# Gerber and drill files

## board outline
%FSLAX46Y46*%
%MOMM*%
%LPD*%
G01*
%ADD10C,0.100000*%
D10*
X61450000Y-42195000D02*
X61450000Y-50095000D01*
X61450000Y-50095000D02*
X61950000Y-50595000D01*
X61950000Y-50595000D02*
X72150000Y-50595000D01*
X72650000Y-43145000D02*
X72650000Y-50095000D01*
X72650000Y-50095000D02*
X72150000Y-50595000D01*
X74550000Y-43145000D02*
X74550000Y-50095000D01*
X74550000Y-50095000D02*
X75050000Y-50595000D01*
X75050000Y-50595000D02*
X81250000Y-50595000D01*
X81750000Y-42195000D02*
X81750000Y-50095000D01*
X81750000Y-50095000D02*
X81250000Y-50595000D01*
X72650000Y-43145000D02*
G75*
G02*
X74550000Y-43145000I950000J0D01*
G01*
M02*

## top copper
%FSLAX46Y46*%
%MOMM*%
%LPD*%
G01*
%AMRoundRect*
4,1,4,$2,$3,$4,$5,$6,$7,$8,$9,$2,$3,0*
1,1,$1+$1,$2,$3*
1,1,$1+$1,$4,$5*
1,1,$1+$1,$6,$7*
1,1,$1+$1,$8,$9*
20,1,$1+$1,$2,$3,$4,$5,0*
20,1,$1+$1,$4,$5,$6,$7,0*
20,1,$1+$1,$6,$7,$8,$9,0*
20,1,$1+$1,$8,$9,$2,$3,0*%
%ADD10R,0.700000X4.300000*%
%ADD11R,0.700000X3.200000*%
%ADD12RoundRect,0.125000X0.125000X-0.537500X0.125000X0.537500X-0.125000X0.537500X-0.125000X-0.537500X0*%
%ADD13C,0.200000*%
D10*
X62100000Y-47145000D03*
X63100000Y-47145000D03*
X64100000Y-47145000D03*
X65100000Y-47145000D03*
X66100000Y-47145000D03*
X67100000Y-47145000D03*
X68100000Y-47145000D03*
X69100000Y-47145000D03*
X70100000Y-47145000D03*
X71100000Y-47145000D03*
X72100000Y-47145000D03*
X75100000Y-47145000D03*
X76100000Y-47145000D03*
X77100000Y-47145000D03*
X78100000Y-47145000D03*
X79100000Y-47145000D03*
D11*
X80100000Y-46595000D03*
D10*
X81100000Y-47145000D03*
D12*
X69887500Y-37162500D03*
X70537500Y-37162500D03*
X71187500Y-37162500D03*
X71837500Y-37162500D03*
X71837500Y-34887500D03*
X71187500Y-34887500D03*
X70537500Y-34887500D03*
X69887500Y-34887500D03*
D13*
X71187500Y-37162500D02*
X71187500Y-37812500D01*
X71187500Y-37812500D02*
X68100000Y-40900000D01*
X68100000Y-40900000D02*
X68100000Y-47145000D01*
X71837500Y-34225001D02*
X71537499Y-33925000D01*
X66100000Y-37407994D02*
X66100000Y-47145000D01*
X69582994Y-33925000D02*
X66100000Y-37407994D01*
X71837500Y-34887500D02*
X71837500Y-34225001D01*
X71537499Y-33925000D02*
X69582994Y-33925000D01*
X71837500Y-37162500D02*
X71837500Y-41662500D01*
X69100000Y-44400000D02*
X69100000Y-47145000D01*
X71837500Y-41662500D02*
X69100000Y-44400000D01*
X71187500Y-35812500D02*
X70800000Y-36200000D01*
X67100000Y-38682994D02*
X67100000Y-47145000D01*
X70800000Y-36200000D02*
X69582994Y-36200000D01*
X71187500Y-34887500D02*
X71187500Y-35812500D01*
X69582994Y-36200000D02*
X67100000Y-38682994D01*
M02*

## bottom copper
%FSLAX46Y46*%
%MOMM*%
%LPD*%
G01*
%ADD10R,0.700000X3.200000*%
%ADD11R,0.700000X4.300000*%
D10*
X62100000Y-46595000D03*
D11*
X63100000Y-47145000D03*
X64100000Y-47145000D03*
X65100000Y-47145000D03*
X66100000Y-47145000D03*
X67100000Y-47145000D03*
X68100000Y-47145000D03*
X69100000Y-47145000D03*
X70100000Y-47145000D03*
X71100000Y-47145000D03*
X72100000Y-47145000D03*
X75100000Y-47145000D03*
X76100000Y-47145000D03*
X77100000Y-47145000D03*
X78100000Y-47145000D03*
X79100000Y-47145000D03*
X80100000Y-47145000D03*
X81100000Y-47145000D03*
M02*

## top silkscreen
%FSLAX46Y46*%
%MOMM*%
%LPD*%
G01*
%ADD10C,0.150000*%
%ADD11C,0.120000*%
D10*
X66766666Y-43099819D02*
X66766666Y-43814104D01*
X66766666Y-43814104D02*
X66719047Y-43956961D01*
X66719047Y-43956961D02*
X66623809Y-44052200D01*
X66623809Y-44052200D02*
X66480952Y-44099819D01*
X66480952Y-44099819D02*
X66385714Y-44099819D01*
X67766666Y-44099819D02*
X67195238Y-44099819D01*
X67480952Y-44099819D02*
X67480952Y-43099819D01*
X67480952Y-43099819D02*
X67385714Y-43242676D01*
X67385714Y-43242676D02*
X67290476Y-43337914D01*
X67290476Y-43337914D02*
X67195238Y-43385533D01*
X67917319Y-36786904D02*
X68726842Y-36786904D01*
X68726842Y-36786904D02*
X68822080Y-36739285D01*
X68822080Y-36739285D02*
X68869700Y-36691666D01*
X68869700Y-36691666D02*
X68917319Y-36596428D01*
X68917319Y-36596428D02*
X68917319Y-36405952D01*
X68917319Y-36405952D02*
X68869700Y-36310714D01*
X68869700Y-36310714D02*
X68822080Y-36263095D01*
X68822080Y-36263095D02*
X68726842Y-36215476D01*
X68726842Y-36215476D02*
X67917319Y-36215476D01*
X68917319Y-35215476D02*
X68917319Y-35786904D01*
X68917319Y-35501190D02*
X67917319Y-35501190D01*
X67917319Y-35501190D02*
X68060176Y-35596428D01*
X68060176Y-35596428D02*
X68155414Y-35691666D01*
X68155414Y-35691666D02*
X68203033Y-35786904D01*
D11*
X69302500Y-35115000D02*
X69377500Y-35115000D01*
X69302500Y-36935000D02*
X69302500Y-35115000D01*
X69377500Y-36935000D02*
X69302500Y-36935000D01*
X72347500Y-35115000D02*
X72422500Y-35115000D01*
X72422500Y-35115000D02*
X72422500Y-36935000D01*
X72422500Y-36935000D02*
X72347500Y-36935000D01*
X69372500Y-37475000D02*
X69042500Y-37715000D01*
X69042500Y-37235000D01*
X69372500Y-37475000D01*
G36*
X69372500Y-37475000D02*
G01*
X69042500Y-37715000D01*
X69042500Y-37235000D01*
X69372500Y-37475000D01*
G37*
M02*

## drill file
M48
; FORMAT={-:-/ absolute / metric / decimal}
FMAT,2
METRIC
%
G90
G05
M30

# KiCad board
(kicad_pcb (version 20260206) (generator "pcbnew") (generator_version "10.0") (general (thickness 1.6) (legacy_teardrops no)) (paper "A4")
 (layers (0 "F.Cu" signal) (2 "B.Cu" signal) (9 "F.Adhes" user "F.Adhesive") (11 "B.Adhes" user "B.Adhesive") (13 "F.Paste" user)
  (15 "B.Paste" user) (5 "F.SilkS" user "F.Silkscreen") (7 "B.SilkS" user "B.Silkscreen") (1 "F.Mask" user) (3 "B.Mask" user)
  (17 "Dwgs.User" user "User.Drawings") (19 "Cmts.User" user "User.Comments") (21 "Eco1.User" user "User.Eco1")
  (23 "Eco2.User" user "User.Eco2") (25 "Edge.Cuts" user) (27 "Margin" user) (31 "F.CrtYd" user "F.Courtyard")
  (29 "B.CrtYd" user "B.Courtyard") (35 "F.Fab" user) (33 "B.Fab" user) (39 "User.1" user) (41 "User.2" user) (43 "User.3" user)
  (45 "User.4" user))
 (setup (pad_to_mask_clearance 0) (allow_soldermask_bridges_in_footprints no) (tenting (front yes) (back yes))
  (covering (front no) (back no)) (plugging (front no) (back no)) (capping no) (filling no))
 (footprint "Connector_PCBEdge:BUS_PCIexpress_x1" (layer "F.Cu") (at 62.1 47.145)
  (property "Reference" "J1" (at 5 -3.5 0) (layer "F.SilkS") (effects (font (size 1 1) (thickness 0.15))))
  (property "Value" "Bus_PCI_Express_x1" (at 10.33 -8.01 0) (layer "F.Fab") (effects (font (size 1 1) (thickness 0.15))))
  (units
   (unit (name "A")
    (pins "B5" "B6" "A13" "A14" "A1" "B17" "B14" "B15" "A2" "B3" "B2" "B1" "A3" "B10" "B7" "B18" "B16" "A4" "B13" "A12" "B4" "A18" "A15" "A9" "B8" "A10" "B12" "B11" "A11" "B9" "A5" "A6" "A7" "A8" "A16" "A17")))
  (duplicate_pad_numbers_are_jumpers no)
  (fp_line (start -0.65 -4.95) (end -0.65 2.95) (stroke (width 0.1) (type solid)) (layer "Edge.Cuts"))
  (fp_line (start -0.65 2.95) (end -0.15 3.45) (stroke (width 0.1) (type solid)) (layer "Edge.Cuts"))
  (fp_line (start -0.15 3.45) (end 10.05 3.45) (stroke (width 0.1) (type solid)) (layer "Edge.Cuts"))
  (fp_line (start 10.55 -4) (end 10.55 2.95) (stroke (width 0.1) (type solid)) (layer "Edge.Cuts"))
  (fp_line (start 10.55 2.95) (end 10.05 3.45) (stroke (width 0.1) (type solid)) (layer "Edge.Cuts"))
  (fp_line (start 12.45 -4) (end 12.45 2.95) (stroke (width 0.1) (type solid)) (layer "Edge.Cuts"))
  (fp_line (start 12.45 2.95) (end 12.95 3.45) (stroke (width 0.1) (type solid)) (layer "Edge.Cuts"))
  (fp_line (start 12.95 3.45) (end 19.15 3.45) (stroke (width 0.1) (type solid)) (layer "Edge.Cuts"))
  (fp_line (start 19.65 -4.95) (end 19.65 2.95) (stroke (width 0.1) (type solid)) (layer "Edge.Cuts"))
  (fp_line (start 19.65 2.95) (end 19.15 3.45) (stroke (width 0.1) (type solid)) (layer "Edge.Cuts"))
  (fp_arc (start 10.55 -4) (mid 11.5 -4.95) (end 12.45 -4) (stroke (width 0.1) (type solid)) (layer "Edge.Cuts"))
  (pad "A1" connect rect (at 0 -0.55) (size 0.7 3.2) (layers "B.Cu" "B.Mask") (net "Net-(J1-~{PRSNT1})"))
  (pad "A2" connect rect (at 1 0) (size 0.7 4.3) (layers "B.Cu" "B.Mask") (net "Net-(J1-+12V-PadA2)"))
  (pad "A3" connect rect (at 2 0) (size 0.7 4.3) (layers "B.Cu" "B.Mask") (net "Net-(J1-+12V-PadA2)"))
  (pad "A4" connect rect (at 3 0) (size 0.7 4.3) (layers "B.Cu" "B.Mask") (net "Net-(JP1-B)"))
  (pad "A5" connect rect (at 4 0) (size 0.7 4.3) (layers "B.Cu" "B.Mask") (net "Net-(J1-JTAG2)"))
  (pad "A6" connect rect (at 5 0) (size 0.7 4.3) (layers "B.Cu" "B.Mask") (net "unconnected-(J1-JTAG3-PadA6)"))
  (pad "A7" connect rect (at 6 0) (size 0.7 4.3) (layers "B.Cu" "B.Mask") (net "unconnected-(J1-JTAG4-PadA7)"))
  (pad "A8" connect rect (at 7 0) (size 0.7 4.3) (layers "B.Cu" "B.Mask") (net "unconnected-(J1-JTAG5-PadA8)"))
  (pad "A9" connect rect (at 8 0) (size 0.7 4.3) (layers "B.Cu" "B.Mask") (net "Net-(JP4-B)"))
  (pad "A10" connect rect (at 9 0) (size 0.7 4.3) (layers "B.Cu" "B.Mask") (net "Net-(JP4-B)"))
  (pad "A11" connect rect (at 10 0) (size 0.7 4.3) (layers "B.Cu" "B.Mask") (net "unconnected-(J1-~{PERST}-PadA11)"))
  (pad "A12" connect rect (at 13 0) (size 0.7 4.3) (layers "B.Cu" "B.Mask") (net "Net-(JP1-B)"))
  (pad "A13" connect rect (at 14 0) (size 0.7 4.3) (layers "B.Cu" "B.Mask") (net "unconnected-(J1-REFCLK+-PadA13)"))
  (pad "A14" connect rect (at 15 0) (size 0.7 4.3) (layers "B.Cu" "B.Mask") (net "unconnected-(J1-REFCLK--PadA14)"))
  (pad "A15" connect rect (at 16 0) (size 0.7 4.3) (layers "B.Cu" "B.Mask") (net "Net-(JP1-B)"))
  (pad "A16" connect rect (at 17 0) (size 0.7 4.3) (layers "B.Cu" "B.Mask") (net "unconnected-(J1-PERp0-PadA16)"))
  (pad "A17" connect rect (at 18 0) (size 0.7 4.3) (layers "B.Cu" "B.Mask") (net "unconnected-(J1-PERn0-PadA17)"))
  (pad "A18" connect rect (at 19 0) (size 0.7 4.3) (layers "B.Cu" "B.Mask") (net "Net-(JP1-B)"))
  (pad "B1" connect rect (at 0 0) (size 0.7 4.3) (layers "F.Cu" "F.Mask") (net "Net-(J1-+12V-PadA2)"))
  (pad "B2" connect rect (at 1 0) (size 0.7 4.3) (layers "F.Cu" "F.Mask") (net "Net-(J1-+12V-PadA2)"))
  (pad "B3" connect rect (at 2 0) (size 0.7 4.3) (layers "F.Cu" "F.Mask") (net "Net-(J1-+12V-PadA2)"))
  (pad "B4" connect rect (at 3 0) (size 0.7 4.3) (layers "F.Cu" "F.Mask") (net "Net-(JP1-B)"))
  (pad "B5" connect rect (at 4 0) (size 0.7 4.3) (layers "F.Cu" "F.Mask") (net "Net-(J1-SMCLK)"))
  (pad "B6" connect rect (at 5 0) (size 0.7 4.3) (layers "F.Cu" "F.Mask") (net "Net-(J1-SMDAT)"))
  (pad "B7" connect rect (at 6 0) (size 0.7 4.3) (layers "F.Cu" "F.Mask") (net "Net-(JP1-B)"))
  (pad "B8" connect rect (at 7 0) (size 0.7 4.3) (layers "F.Cu" "F.Mask") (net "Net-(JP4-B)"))
  (pad "B9" connect rect (at 8 0) (size 0.7 4.3) (layers "F.Cu" "F.Mask") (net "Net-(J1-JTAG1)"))
  (pad "B10" connect rect (at 9 0) (size 0.7 4.3) (layers "F.Cu" "F.Mask") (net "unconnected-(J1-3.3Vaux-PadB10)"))
  (pad "B11" connect rect (at 10 0) (size 0.7 4.3) (layers "F.Cu" "F.Mask") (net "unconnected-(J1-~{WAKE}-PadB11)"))
  (pad "B12" connect rect (at 13 0) (size 0.7 4.3) (layers "F.Cu" "F.Mask") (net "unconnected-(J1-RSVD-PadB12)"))
  (pad "B13" connect rect (at 14 0) (size 0.7 4.3) (layers "F.Cu" "F.Mask") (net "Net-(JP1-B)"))
  (pad "B14" connect rect (at 15 0) (size 0.7 4.3) (layers "F.Cu" "F.Mask") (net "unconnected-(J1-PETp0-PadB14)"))
  (pad "B15" connect rect (at 16 0) (size 0.7 4.3) (layers "F.Cu" "F.Mask") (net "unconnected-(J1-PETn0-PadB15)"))
  (pad "B16" connect rect (at 17 0) (size 0.7 4.3) (layers "F.Cu" "F.Mask") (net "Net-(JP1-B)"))
  (pad "B17" connect rect (at 18 -0.55) (size 0.7 3.2) (layers "F.Cu" "F.Mask") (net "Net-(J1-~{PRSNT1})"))
  (pad "B18" connect rect (at 19 0) (size 0.7 4.3) (layers "F.Cu" "F.Mask") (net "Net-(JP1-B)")))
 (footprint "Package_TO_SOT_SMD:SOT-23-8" (layer "F.Cu") (at 70.8625 36.025 90)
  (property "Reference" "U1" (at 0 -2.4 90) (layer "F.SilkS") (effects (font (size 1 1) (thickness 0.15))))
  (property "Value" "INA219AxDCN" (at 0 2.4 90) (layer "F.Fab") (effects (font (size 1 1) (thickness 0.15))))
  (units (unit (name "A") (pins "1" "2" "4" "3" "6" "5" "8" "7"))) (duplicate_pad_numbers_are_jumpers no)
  (fp_line (start 0.91 -1.56) (end 0.91 -1.485) (stroke (width 0.12) (type solid)) (layer "F.SilkS"))
  (fp_line (start -0.91 -1.56) (end 0.91 -1.56) (stroke (width 0.12) (type solid)) (layer "F.SilkS"))
  (fp_line (start -0.91 -1.485) (end -0.91 -1.56) (stroke (width 0.12) (type solid)) (layer "F.SilkS"))
  (fp_line (start 0.91 1.485) (end 0.91 1.56) (stroke (width 0.12) (type solid)) (layer "F.SilkS"))
  (fp_line (start 0.91 1.56) (end -0.91 1.56) (stroke (width 0.12) (type solid)) (layer "F.SilkS"))
  (fp_line (start -0.91 1.56) (end -0.91 1.485) (stroke (width 0.12) (type solid)) (layer "F.SilkS"))
  (fp_poly (pts (xy -1.45 -1.49) (xy -1.69 -1.82) (xy -1.21 -1.82)) (stroke (width 0.12) (type solid)) (fill yes) (layer "F.SilkS"))
  (pad "1" smd roundrect (at -1.1375 -0.975 90) (size 1.325 0.5) (layers "F.Cu" "F.Mask" "F.Paste") (roundrect_rratio 0.25)
   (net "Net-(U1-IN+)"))
  (pad "2" smd roundrect (at -1.1375 -0.325 90) (size 1.325 0.5) (layers "F.Cu" "F.Mask" "F.Paste") (roundrect_rratio 0.25)
   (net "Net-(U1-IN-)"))
  (pad "3" smd roundrect (at -1.1375 0.325 90) (size 1.325 0.5) (layers "F.Cu" "F.Mask" "F.Paste") (roundrect_rratio 0.25)
   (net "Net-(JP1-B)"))
  (pad "4" smd roundrect (at -1.1375 0.975 90) (size 1.325 0.5) (layers "F.Cu" "F.Mask" "F.Paste") (roundrect_rratio 0.25)
   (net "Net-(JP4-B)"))
  (pad "5" smd roundrect (at 1.1375 0.975 90) (size 1.325 0.5) (layers "F.Cu" "F.Mask" "F.Paste") (roundrect_rratio 0.25)
   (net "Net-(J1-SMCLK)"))
  (pad "6" smd roundrect (at 1.1375 0.325 90) (size 1.325 0.5) (layers "F.Cu" "F.Mask" "F.Paste") (roundrect_rratio 0.25)
   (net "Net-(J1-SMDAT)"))
  (pad "7" smd roundrect (at 1.1375 -0.325 90) (size 1.325 0.5) (layers "F.Cu" "F.Mask" "F.Paste") (roundrect_rratio 0.25)
   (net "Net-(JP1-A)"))
  (pad "8" smd roundrect (at 1.1375 -0.975 90) (size 1.325 0.5) (layers "F.Cu" "F.Mask" "F.Paste") (roundrect_rratio 0.25)
   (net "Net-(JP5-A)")))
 (segment (start 71.1875 37.1625) (end 71.1875 37.8125) (width 0.2) (layer "F.Cu") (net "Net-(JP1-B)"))
 (segment (start 71.1875 37.8125) (end 68.1 40.9) (width 0.2) (layer "F.Cu") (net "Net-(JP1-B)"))
 (segment (start 68.1 40.9) (end 68.1 47.145) (width 0.2) (layer "F.Cu") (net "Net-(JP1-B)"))
 (segment (start 71.8375 34.225001) (end 71.537499 33.925) (width 0.2) (layer "F.Cu") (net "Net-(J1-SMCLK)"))
 (segment (start 66.1 37.407994) (end 66.1 47.145) (width 0.2) (layer "F.Cu") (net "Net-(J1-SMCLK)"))
 (segment (start 69.582994 33.925) (end 66.1 37.407994) (width 0.2) (layer "F.Cu") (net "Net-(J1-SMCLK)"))
 (segment (start 71.8375 34.8875) (end 71.8375 34.225001) (width 0.2) (layer "F.Cu") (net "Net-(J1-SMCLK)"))
 (segment (start 71.537499 33.925) (end 69.582994 33.925) (width 0.2) (layer "F.Cu") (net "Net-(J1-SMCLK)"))
 (segment (start 71.8375 37.1625) (end 71.8375 41.6625) (width 0.2) (layer "F.Cu") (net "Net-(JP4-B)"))
 (segment (start 69.1 44.4) (end 69.1 47.145) (width 0.2) (layer "F.Cu") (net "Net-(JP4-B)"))
 (segment (start 71.8375 41.6625) (end 69.1 44.4) (width 0.2) (layer "F.Cu") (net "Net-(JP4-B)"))
 (segment (start 71.1875 35.8125) (end 70.8 36.2) (width 0.2) (layer "F.Cu") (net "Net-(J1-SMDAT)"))
 (segment (start 67.1 38.682994) (end 67.1 47.145) (width 0.2) (layer "F.Cu") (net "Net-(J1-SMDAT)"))
 (segment (start 70.8 36.2) (end 69.582994 36.2) (width 0.2) (layer "F.Cu") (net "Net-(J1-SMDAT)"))
 (segment (start 71.1875 34.8875) (end 71.1875 35.8125) (width 0.2) (layer "F.Cu") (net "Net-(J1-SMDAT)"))
 (segment (start 69.582994 36.2) (end 67.1 38.682994) (width 0.2) (layer "F.Cu") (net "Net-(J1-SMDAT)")))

